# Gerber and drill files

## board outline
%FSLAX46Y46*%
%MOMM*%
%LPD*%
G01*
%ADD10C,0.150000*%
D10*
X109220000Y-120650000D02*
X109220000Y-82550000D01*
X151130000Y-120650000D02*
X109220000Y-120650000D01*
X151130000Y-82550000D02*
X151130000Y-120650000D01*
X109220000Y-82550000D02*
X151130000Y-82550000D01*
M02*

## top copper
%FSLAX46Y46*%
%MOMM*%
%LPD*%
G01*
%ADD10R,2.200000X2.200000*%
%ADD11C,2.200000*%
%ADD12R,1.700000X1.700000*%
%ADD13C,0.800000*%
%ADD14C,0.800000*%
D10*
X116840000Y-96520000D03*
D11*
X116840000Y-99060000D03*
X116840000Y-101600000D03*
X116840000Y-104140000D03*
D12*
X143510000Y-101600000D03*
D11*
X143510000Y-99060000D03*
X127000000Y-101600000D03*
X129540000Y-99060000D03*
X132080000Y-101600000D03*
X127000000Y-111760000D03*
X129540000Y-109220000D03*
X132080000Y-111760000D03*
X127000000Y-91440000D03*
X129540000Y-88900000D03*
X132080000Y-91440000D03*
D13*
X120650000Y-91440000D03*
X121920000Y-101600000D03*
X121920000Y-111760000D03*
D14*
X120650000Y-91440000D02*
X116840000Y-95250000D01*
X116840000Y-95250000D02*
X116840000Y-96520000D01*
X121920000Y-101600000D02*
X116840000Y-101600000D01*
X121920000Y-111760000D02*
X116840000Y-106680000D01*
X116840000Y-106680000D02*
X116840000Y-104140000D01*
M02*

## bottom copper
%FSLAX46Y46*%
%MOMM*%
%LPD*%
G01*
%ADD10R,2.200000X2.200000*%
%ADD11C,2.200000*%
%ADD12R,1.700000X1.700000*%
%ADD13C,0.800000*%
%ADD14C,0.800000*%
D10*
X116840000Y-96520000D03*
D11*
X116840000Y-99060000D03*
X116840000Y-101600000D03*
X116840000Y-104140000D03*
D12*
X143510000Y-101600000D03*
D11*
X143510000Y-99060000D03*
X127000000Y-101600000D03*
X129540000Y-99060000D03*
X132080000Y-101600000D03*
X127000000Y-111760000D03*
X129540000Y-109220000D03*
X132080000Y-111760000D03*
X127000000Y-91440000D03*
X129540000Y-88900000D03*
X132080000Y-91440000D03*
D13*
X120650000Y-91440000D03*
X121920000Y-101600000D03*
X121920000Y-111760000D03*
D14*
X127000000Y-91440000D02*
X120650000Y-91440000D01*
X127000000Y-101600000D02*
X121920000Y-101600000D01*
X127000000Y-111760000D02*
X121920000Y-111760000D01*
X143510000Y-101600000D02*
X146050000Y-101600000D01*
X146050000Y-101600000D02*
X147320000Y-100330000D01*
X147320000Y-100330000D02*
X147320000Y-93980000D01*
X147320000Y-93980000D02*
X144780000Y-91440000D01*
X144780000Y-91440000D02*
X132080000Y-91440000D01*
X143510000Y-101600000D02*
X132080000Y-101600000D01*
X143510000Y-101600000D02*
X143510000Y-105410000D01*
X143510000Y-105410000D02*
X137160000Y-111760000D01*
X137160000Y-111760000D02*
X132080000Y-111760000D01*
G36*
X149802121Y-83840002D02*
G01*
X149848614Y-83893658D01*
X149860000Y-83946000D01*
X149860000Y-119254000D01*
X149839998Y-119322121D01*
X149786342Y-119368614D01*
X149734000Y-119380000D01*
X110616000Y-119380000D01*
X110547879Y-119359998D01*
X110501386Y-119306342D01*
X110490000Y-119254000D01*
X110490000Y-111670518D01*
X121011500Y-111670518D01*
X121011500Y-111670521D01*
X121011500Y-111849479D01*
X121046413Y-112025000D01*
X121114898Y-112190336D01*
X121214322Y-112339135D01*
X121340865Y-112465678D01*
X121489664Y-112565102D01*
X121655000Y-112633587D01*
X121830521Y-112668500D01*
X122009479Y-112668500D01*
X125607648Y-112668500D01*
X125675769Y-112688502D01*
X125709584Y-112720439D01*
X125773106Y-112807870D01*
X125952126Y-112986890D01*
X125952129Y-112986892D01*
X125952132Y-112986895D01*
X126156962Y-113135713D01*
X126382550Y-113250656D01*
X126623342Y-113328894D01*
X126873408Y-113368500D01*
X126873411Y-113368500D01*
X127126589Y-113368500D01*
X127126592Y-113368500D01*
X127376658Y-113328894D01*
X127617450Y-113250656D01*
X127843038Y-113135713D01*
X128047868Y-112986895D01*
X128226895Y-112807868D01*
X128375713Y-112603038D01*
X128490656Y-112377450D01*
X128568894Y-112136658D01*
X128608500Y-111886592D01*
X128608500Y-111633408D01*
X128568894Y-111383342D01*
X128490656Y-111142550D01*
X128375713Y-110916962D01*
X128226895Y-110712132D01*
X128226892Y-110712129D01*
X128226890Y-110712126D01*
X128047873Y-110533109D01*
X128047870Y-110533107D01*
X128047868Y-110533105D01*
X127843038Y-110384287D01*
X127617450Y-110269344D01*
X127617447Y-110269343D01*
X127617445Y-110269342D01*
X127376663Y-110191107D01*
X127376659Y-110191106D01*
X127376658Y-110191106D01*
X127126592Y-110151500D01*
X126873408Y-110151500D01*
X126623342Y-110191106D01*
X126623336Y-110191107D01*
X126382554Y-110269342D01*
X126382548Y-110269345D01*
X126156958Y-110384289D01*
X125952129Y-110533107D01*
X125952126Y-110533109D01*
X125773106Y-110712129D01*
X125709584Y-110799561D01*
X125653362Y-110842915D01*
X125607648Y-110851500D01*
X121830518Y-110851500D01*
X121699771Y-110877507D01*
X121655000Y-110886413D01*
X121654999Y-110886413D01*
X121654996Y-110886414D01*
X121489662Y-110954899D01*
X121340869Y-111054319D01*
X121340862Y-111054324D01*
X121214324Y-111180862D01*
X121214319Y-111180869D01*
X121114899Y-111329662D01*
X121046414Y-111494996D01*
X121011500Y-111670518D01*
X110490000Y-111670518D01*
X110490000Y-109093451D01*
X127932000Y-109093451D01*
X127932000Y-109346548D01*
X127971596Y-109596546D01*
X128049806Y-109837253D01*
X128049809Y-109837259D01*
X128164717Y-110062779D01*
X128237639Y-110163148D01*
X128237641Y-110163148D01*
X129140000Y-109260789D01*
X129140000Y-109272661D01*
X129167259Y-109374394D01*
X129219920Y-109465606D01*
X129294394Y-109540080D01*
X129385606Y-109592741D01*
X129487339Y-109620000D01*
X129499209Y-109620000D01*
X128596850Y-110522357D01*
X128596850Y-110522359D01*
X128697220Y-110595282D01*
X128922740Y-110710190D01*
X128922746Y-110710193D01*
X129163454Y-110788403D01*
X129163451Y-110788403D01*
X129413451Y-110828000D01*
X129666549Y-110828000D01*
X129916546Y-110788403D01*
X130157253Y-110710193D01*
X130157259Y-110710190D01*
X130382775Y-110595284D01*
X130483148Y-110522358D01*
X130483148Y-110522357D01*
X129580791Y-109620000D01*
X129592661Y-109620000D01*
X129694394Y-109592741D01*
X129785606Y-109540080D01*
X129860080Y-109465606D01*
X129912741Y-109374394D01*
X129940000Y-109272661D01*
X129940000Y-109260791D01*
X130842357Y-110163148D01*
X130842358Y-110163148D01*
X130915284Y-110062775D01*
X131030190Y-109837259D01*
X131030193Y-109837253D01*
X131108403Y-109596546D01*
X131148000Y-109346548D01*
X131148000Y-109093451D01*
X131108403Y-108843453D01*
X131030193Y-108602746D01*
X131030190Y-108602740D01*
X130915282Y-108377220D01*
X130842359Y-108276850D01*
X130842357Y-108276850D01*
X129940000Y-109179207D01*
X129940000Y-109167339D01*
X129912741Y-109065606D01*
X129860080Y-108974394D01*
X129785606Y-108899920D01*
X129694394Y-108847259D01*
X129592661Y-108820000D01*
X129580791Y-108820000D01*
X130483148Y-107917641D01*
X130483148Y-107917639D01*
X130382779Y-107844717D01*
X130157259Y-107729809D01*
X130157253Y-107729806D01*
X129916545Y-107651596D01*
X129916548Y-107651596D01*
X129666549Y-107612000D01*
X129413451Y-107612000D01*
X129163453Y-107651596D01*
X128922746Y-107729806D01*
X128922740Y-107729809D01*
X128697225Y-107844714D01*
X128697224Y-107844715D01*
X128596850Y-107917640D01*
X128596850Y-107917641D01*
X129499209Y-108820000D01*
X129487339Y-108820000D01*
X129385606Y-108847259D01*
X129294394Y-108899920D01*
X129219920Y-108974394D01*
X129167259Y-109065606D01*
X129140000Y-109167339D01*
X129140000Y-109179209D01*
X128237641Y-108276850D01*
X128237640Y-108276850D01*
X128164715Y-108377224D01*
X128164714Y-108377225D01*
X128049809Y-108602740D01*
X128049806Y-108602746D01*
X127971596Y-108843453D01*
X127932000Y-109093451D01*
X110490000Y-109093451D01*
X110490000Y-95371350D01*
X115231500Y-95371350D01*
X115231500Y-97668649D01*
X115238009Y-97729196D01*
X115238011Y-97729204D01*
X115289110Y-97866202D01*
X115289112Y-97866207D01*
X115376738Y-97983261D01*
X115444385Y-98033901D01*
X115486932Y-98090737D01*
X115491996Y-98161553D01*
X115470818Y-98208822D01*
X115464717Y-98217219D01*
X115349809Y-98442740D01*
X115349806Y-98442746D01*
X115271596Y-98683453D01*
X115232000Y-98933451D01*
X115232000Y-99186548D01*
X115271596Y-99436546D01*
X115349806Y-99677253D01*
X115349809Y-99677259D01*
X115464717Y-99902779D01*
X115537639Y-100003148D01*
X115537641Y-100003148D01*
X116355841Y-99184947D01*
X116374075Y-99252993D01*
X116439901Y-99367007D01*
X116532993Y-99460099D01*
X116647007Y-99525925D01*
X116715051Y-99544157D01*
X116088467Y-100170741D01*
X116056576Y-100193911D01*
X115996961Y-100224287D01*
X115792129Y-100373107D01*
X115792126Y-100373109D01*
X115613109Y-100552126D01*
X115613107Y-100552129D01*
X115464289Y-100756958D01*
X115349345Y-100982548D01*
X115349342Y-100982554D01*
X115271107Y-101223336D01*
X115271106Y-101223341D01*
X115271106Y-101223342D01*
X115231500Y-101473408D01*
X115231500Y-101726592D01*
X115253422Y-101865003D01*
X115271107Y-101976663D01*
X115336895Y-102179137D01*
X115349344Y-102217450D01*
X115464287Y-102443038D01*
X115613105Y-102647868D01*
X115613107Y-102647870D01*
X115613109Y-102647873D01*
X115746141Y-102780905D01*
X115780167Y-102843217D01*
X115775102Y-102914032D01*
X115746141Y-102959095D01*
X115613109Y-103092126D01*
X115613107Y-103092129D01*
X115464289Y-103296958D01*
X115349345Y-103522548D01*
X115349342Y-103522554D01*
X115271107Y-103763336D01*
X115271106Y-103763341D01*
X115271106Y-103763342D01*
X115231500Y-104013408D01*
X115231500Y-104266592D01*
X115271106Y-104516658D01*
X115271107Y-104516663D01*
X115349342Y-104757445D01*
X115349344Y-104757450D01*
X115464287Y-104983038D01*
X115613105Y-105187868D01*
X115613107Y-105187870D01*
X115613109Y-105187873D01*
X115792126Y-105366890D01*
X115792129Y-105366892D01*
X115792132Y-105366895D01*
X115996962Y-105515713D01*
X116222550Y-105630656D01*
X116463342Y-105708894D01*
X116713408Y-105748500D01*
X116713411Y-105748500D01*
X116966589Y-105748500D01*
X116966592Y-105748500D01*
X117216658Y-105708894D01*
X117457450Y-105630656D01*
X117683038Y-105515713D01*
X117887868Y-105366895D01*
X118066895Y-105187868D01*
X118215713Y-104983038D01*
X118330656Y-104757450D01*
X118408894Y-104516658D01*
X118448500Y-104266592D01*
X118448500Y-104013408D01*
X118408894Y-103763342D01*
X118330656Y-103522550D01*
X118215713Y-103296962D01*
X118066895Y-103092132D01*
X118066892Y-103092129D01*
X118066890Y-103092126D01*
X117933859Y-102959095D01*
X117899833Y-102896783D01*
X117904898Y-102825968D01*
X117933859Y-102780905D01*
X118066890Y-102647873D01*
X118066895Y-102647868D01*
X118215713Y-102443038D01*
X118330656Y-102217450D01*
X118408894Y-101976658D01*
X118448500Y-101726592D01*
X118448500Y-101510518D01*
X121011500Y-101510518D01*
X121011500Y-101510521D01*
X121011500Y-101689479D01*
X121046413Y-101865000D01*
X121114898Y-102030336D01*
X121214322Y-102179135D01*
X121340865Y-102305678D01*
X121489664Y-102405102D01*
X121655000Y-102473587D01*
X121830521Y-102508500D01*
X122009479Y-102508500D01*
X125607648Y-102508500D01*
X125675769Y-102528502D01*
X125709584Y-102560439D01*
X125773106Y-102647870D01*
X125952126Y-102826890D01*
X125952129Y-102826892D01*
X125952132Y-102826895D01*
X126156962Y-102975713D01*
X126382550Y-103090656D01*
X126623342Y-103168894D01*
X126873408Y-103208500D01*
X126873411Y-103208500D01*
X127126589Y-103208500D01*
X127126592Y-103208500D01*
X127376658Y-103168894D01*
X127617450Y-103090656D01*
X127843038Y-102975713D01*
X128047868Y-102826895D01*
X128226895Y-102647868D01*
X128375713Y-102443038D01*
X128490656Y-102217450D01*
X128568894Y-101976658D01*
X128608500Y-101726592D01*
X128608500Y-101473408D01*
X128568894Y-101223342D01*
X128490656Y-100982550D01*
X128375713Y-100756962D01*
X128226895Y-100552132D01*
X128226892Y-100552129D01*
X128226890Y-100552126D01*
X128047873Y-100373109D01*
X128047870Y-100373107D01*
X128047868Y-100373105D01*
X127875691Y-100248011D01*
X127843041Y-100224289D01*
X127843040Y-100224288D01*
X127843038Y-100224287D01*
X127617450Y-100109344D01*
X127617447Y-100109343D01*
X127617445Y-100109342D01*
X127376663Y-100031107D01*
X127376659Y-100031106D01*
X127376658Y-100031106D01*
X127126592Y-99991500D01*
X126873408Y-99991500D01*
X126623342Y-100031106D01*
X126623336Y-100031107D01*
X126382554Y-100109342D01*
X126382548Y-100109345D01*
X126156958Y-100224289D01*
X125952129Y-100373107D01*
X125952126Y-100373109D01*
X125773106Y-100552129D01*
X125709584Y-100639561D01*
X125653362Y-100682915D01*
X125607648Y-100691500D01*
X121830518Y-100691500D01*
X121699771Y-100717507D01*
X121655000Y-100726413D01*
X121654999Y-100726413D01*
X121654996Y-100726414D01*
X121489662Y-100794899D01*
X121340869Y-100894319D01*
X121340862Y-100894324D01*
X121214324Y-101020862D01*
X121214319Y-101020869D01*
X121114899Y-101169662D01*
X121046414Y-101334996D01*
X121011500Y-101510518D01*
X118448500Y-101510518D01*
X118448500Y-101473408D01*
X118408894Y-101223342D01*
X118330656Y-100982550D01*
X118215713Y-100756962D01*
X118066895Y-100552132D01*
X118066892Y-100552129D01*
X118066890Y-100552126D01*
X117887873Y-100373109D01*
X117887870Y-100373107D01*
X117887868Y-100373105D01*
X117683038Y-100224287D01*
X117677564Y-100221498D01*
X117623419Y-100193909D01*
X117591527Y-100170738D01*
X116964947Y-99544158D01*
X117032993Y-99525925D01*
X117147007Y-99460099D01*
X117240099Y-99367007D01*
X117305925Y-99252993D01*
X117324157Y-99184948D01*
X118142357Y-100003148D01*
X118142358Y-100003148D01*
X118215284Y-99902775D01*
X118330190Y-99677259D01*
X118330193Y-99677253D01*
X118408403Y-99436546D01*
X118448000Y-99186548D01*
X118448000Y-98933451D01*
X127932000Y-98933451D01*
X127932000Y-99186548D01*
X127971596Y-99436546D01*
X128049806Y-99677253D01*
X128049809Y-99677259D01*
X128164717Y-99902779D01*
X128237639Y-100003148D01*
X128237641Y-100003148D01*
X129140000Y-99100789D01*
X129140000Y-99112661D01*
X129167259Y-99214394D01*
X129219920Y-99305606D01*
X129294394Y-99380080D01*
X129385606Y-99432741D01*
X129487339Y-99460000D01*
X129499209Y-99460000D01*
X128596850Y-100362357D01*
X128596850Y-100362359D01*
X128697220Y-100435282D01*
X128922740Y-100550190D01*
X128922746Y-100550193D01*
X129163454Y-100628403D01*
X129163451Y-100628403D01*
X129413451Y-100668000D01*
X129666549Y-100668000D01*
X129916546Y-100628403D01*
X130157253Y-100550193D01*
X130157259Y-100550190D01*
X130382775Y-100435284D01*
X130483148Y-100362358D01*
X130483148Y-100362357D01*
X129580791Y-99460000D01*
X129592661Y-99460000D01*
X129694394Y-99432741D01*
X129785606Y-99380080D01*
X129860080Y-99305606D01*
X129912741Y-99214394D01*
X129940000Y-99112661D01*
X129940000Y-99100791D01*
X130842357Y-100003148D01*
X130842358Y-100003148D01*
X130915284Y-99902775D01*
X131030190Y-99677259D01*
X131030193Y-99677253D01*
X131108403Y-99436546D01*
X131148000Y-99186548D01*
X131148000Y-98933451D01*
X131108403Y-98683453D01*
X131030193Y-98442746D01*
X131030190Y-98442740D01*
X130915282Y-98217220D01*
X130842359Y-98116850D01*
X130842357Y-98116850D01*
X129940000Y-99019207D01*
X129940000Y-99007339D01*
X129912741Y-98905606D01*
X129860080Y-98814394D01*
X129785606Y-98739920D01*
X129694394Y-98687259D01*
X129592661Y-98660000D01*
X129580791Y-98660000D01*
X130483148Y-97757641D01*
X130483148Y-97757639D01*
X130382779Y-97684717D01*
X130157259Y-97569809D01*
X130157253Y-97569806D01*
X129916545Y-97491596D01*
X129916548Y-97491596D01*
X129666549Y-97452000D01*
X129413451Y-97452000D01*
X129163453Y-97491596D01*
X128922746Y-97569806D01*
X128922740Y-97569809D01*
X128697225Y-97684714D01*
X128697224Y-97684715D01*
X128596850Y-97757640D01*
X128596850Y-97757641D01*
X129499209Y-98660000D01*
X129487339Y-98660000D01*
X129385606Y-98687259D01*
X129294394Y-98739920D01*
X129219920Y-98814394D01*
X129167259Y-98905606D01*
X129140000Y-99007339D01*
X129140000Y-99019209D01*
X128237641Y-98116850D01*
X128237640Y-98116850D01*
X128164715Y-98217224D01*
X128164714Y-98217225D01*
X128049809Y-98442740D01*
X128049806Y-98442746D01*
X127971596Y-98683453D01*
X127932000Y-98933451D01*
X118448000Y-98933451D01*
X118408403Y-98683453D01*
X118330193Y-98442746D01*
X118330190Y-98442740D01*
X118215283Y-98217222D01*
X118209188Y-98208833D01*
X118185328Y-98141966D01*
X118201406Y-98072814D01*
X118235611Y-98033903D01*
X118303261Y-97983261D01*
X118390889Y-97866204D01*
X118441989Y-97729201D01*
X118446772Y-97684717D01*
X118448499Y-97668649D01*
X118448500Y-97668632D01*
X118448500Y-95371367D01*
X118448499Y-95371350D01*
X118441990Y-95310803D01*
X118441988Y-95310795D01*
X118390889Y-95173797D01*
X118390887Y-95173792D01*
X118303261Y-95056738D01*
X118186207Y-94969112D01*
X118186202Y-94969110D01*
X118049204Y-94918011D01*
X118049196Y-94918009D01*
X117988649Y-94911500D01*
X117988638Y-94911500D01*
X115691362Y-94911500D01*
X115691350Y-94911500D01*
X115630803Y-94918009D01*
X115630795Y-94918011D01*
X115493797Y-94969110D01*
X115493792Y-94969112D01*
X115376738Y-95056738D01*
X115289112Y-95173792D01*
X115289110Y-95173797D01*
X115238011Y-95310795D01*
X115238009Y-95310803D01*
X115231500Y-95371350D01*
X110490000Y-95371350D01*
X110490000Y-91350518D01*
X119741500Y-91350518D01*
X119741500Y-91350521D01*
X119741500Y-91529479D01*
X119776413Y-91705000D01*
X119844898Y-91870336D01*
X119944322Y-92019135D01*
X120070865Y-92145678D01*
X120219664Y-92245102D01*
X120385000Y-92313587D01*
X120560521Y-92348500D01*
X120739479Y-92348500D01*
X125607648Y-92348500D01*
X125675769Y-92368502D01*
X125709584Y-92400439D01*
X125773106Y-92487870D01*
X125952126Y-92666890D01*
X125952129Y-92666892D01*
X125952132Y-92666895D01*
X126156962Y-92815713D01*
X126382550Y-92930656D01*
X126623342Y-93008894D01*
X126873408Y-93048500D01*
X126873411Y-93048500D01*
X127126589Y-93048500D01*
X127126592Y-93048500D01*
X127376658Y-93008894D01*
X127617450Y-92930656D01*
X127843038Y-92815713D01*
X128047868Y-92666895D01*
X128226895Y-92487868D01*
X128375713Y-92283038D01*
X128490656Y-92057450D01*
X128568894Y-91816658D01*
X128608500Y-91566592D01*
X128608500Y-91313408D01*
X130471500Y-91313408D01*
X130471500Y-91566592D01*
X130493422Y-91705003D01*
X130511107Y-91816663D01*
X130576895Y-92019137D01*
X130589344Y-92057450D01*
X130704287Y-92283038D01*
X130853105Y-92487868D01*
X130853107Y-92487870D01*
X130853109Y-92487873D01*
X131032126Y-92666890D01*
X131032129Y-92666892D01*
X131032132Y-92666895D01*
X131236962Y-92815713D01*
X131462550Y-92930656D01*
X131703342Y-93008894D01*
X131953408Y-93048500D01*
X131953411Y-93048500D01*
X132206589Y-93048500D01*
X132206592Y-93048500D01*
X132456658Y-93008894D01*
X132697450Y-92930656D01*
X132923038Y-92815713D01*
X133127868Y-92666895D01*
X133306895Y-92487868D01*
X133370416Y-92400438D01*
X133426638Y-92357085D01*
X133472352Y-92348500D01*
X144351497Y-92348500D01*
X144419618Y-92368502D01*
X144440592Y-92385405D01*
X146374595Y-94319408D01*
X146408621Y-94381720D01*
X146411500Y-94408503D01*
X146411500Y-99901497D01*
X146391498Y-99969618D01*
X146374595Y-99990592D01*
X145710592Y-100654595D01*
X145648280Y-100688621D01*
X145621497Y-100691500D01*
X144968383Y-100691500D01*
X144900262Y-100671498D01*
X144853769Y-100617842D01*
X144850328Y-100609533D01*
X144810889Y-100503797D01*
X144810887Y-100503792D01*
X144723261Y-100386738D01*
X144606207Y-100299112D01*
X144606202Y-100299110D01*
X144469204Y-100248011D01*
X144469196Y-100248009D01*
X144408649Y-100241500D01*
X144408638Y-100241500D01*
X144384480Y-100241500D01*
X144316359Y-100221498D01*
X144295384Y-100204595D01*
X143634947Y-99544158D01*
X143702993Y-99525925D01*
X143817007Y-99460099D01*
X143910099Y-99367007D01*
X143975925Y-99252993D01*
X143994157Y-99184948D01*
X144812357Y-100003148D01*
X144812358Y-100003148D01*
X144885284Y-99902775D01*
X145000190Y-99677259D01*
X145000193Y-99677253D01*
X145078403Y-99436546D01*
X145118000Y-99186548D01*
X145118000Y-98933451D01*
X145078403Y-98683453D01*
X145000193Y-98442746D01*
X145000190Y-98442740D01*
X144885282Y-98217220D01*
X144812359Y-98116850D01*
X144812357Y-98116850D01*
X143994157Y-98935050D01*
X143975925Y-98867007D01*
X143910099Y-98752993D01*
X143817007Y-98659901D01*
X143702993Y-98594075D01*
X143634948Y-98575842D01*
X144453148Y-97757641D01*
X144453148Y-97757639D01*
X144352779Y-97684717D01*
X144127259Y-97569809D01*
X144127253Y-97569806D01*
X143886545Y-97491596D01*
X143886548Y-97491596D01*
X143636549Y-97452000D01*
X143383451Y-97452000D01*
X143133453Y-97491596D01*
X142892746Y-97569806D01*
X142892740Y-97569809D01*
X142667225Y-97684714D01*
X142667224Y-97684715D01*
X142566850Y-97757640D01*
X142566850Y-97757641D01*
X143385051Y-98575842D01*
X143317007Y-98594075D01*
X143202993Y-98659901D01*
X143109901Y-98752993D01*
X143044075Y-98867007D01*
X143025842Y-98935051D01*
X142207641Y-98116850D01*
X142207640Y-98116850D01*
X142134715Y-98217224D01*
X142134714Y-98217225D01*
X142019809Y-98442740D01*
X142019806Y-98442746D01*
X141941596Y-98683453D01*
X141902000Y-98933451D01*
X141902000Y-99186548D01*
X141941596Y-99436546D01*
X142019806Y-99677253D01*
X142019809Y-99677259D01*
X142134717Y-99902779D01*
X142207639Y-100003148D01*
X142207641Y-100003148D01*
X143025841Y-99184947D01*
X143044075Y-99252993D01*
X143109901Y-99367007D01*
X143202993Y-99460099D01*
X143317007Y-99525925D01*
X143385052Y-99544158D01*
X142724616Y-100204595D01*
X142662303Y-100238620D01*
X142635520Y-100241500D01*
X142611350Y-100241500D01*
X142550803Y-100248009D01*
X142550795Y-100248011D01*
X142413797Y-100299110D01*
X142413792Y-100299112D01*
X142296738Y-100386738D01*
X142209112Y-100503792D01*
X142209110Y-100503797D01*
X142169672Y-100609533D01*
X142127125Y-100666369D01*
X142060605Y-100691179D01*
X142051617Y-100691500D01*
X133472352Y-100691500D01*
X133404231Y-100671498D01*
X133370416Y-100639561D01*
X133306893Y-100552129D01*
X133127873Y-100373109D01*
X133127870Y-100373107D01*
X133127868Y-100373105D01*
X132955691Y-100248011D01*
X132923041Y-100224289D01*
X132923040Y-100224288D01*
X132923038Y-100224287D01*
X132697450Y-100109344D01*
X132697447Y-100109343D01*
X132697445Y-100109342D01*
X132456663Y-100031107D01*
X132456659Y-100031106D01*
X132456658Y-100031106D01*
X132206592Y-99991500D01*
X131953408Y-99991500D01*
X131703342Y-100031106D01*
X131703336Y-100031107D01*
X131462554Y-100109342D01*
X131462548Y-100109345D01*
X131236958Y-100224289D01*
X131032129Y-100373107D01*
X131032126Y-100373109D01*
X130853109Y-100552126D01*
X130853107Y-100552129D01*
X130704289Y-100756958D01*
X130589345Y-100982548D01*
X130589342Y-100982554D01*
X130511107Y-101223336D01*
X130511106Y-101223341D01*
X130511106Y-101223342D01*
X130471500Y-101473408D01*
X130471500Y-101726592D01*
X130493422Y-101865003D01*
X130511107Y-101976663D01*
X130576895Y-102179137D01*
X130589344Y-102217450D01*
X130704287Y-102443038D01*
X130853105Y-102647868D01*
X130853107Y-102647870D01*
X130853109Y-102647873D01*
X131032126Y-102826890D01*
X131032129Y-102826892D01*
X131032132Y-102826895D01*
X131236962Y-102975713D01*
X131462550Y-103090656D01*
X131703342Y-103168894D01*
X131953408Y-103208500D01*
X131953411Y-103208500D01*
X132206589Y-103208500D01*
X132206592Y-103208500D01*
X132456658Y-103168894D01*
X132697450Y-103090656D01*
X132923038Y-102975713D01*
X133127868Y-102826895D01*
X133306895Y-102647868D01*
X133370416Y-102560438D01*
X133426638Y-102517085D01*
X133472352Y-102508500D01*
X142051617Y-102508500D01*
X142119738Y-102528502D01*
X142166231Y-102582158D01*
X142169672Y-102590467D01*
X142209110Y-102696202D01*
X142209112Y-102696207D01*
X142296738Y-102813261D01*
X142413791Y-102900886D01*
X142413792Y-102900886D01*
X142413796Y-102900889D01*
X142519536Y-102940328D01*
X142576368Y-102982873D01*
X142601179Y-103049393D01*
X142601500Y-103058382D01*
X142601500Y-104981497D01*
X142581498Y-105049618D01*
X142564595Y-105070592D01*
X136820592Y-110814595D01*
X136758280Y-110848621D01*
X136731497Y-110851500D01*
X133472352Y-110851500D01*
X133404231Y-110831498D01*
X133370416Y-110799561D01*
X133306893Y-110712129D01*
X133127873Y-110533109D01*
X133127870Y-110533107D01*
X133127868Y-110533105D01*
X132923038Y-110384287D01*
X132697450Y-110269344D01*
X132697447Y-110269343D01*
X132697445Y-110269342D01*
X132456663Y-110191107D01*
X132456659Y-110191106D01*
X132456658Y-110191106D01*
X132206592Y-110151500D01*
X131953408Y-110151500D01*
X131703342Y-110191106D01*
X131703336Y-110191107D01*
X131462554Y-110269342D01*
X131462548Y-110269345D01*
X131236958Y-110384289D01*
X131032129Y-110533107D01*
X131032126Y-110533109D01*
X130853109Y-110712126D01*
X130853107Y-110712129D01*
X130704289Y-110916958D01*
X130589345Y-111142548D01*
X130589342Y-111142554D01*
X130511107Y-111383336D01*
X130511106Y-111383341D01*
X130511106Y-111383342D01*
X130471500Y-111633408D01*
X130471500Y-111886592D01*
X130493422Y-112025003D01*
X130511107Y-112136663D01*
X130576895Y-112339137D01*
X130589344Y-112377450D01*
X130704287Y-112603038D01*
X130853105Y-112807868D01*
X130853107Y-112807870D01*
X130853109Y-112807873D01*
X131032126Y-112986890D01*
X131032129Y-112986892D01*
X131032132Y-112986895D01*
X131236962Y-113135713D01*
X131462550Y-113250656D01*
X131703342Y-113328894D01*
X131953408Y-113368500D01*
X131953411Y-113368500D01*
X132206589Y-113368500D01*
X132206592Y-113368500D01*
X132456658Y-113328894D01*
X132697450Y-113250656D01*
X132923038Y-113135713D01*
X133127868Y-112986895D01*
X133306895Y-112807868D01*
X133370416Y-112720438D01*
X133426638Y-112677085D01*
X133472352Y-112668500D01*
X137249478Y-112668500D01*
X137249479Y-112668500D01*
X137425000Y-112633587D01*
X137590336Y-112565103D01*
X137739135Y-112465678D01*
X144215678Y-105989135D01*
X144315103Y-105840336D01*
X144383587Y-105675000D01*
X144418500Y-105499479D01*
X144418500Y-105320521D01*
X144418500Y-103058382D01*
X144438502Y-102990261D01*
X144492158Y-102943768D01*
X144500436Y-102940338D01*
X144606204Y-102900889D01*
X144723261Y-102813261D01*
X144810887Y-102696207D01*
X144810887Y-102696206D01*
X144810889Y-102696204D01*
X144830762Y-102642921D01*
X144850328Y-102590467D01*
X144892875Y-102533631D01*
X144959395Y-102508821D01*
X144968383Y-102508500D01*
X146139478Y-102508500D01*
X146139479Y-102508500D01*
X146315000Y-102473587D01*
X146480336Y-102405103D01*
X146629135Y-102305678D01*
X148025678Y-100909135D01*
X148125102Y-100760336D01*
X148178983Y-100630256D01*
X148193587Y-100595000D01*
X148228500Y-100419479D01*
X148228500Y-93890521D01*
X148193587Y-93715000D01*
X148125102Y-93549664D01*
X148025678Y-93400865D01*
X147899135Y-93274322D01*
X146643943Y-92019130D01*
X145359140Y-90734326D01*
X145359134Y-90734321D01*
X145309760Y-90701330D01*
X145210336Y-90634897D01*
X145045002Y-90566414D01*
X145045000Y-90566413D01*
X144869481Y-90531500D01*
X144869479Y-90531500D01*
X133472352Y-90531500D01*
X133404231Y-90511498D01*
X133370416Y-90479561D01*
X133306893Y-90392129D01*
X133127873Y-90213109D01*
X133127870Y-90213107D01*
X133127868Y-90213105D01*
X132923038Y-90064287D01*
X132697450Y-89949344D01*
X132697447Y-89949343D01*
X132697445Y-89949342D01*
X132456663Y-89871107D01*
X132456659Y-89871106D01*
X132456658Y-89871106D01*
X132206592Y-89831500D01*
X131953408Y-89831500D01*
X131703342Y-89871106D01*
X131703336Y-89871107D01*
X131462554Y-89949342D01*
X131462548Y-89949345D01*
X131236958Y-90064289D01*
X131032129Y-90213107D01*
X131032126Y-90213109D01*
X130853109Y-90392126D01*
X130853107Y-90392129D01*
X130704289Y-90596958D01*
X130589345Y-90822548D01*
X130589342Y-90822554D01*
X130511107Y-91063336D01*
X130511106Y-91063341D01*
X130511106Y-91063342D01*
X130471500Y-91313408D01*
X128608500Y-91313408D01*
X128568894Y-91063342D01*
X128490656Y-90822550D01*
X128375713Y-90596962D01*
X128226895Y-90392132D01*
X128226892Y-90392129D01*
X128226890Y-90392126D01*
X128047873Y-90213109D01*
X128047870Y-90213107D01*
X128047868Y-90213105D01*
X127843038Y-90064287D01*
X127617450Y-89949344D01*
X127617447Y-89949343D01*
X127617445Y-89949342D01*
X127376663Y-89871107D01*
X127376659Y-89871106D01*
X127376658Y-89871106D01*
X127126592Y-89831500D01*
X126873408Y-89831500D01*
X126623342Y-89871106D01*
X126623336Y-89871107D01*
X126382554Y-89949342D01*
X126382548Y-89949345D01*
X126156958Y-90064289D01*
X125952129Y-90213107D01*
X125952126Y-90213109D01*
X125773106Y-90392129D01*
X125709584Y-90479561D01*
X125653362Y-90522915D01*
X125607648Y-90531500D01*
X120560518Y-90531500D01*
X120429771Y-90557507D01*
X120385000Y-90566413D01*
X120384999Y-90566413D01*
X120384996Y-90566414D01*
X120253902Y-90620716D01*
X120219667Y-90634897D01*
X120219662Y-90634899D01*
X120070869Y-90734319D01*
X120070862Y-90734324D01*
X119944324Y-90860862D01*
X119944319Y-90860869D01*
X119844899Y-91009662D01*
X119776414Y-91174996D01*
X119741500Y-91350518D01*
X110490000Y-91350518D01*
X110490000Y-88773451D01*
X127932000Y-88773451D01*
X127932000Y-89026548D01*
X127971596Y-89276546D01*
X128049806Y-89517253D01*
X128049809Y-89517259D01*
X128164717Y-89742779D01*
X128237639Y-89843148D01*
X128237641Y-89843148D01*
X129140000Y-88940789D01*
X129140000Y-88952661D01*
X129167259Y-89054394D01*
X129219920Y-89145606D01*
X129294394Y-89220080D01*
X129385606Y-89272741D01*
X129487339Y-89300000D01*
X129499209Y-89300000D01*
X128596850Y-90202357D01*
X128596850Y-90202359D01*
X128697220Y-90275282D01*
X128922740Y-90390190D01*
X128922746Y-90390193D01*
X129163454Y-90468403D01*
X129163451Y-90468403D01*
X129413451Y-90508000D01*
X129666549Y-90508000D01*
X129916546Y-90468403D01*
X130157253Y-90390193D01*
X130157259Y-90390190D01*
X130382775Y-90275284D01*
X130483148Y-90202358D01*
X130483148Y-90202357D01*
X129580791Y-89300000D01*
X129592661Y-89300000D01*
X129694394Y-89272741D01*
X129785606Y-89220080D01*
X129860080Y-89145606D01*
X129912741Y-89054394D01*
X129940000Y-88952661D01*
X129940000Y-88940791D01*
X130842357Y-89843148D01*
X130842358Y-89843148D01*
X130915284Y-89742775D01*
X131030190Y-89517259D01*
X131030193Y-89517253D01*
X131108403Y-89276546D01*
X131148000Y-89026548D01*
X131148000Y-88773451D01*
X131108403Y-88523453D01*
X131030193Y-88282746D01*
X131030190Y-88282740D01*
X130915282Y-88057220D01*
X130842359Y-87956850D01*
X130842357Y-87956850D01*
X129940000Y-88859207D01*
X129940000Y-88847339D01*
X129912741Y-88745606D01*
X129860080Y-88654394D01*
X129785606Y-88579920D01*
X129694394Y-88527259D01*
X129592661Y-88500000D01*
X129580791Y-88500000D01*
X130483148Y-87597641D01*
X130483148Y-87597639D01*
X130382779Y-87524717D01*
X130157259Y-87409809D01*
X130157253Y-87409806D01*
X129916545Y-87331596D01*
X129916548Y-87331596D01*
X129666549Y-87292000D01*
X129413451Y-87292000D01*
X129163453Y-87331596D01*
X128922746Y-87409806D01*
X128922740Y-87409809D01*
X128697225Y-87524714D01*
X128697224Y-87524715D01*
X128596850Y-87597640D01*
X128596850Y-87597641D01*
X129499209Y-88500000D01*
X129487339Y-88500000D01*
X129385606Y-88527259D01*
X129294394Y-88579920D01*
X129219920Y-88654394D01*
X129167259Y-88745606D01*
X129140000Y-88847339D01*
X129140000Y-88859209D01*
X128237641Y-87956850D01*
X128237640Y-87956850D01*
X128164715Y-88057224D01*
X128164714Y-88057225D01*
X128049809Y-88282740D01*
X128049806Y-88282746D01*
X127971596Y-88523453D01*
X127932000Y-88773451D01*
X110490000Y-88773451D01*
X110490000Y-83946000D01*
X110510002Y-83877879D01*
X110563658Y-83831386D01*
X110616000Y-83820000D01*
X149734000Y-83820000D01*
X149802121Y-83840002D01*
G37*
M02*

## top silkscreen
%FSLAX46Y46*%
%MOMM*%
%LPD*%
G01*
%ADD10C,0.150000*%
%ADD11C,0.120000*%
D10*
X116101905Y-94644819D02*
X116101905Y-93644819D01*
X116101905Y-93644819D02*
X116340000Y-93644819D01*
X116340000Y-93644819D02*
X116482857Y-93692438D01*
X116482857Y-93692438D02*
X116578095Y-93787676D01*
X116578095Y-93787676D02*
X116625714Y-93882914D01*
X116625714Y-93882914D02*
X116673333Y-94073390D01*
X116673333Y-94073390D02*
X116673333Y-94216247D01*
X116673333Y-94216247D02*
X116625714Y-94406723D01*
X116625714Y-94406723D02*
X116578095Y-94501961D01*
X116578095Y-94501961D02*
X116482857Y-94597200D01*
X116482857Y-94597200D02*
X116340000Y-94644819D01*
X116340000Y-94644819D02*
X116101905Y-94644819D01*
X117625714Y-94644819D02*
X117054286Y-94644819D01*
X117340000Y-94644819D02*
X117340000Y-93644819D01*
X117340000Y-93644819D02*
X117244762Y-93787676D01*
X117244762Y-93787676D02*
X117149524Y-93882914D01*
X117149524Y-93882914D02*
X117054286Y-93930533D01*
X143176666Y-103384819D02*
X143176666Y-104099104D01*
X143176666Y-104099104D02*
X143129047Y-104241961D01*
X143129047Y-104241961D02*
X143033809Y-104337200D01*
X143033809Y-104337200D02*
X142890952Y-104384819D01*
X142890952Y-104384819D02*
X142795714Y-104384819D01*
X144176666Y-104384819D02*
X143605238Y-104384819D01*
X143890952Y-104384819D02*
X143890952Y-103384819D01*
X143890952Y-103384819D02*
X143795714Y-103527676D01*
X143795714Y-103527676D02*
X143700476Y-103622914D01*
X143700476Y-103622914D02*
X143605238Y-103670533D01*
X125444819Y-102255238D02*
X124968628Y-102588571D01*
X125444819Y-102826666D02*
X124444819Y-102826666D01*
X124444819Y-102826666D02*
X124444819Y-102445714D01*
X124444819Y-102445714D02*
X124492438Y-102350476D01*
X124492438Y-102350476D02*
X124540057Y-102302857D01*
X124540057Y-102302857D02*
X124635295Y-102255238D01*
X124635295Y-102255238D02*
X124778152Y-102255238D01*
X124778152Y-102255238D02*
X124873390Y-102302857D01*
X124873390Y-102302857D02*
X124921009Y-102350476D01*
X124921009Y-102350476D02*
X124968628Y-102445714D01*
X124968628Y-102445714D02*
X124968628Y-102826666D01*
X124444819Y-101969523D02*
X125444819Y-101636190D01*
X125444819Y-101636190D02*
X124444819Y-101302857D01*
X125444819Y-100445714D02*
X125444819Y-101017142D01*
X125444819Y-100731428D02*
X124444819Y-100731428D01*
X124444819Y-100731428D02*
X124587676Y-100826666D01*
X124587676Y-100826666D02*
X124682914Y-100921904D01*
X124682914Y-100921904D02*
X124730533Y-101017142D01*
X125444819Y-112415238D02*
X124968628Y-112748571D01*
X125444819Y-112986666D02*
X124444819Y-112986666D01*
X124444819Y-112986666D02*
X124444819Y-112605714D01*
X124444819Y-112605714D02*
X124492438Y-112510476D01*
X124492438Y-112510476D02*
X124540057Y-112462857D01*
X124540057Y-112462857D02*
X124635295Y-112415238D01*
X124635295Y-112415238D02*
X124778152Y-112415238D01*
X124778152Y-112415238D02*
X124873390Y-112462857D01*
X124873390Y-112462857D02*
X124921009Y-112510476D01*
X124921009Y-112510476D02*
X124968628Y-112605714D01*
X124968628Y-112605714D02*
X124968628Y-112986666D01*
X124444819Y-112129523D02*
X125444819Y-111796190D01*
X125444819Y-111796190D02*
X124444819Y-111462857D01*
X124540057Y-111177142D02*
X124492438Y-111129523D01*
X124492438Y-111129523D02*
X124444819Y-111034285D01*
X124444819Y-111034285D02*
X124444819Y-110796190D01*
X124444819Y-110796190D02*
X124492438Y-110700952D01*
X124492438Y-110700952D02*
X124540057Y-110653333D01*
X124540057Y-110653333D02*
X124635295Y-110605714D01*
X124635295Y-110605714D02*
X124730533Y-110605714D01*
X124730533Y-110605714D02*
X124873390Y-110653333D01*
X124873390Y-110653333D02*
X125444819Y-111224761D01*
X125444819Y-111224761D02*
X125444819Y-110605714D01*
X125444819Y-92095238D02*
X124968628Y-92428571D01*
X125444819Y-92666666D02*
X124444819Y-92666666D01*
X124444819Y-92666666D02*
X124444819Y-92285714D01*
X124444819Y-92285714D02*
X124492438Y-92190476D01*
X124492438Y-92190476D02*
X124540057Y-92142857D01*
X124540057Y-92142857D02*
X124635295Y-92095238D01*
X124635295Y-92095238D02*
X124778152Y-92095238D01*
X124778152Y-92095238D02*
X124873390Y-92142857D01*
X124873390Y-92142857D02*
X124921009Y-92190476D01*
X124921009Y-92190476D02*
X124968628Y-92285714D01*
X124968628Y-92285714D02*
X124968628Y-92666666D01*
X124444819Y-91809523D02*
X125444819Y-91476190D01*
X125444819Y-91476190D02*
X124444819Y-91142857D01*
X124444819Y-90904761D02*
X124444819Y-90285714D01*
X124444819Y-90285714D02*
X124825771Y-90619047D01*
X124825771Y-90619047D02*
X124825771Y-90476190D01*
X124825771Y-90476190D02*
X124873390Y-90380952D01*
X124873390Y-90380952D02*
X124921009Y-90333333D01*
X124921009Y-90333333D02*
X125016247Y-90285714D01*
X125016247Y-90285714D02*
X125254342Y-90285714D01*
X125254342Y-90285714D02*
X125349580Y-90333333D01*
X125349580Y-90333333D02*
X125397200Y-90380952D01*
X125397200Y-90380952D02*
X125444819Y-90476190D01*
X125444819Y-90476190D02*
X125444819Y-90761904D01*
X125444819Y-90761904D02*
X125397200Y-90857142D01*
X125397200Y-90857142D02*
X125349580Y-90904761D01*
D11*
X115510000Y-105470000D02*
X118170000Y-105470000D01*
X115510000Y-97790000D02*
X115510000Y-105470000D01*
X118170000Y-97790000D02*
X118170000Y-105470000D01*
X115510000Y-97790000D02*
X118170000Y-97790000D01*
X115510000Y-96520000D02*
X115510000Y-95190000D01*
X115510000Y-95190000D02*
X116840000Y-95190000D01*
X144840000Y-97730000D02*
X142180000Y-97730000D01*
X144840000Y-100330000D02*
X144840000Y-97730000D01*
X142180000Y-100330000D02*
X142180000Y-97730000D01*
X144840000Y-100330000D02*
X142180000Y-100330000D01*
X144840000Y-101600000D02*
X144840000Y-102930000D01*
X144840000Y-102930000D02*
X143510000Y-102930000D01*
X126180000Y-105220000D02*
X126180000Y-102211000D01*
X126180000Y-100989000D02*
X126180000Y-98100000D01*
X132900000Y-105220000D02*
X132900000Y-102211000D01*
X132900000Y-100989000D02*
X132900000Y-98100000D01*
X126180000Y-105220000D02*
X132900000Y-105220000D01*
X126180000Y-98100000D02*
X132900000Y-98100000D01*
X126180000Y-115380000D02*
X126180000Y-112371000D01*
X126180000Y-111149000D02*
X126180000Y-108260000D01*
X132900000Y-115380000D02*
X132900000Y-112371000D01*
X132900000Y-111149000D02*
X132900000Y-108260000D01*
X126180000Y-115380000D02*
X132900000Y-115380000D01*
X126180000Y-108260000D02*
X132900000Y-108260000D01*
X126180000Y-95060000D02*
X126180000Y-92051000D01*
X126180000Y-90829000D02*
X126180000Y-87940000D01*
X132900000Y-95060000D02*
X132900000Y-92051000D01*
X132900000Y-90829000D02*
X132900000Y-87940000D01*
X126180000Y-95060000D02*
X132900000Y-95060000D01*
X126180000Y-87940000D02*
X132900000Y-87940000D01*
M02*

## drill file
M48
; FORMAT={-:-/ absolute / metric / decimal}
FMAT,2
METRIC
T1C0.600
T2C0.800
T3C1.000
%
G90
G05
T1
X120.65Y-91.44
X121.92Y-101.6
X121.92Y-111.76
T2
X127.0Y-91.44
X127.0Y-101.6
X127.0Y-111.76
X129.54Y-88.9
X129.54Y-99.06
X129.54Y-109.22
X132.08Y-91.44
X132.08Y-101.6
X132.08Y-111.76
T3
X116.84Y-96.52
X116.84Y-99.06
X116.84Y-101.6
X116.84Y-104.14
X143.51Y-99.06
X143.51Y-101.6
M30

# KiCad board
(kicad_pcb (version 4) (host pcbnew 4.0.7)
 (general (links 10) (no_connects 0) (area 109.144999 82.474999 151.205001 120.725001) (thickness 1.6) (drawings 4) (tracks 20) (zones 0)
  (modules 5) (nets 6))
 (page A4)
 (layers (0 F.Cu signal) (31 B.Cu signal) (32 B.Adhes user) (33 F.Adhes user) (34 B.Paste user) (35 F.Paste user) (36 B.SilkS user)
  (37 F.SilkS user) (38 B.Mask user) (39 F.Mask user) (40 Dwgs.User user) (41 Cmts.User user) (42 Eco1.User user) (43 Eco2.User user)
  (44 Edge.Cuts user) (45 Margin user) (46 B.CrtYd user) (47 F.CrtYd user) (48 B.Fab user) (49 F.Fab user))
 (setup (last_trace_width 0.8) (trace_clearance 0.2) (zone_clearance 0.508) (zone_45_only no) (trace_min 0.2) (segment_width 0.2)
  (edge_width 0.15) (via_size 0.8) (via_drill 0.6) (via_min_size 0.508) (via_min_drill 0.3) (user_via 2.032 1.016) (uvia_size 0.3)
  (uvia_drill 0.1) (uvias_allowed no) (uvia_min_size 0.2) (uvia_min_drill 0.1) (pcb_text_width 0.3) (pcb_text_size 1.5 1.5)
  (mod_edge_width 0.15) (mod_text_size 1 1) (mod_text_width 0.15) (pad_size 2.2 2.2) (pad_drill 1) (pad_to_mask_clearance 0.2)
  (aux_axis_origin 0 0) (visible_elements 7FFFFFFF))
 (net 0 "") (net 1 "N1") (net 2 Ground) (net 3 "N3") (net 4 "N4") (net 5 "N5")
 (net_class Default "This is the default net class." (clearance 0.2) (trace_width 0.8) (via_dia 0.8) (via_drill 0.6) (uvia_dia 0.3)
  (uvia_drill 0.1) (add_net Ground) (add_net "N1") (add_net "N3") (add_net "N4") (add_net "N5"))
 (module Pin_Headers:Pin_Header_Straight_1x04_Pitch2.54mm (layer F.Cu) (at 116.84 96.52)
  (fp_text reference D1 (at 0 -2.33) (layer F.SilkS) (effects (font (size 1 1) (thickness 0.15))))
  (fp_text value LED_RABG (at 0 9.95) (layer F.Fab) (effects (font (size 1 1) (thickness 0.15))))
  (fp_line (start -1.33 8.95) (end 1.33 8.95) (layer F.SilkS) (width 0.12))
  (fp_line (start -1.33 1.27) (end -1.33 8.95) (layer F.SilkS) (width 0.12))
  (fp_line (start 1.33 1.27) (end 1.33 8.95) (layer F.SilkS) (width 0.12))
  (fp_line (start -1.33 1.27) (end 1.33 1.27) (layer F.SilkS) (width 0.12))
  (fp_line (start -1.33 0) (end -1.33 -1.33) (layer F.SilkS) (width 0.12))
  (fp_line (start -1.33 -1.33) (end 0 -1.33) (layer F.SilkS) (width 0.12))
  (pad 1 thru_hole rect (at 0 0) (size 2.2 2.2) (drill 1) (layers *.Cu *.Mask) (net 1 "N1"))
  (pad 2 thru_hole circle (at 0 2.54) (size 2.2 2.2) (drill 1) (layers *.Cu *.Mask) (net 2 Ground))
  (pad 3 thru_hole circle (at 0 5.08) (size 2.2 2.2) (drill 1) (layers *.Cu *.Mask) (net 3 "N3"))
  (pad 4 thru_hole circle (at 0 7.62) (size 2.2 2.2) (drill 1) (layers *.Cu *.Mask) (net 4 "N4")))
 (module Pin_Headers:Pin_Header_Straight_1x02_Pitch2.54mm (layer F.Cu) (at 143.51 101.6 180)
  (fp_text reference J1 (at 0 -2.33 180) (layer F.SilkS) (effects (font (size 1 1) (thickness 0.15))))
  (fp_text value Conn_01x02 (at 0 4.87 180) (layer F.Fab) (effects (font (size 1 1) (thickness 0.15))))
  (fp_line (start -1.33 3.87) (end 1.33 3.87) (layer F.SilkS) (width 0.12))
  (fp_line (start -1.33 1.27) (end -1.33 3.87) (layer F.SilkS) (width 0.12))
  (fp_line (start 1.33 1.27) (end 1.33 3.87) (layer F.SilkS) (width 0.12))
  (fp_line (start -1.33 1.27) (end 1.33 1.27) (layer F.SilkS) (width 0.12))
  (fp_line (start -1.33 0) (end -1.33 -1.33) (layer F.SilkS) (width 0.12))
  (fp_line (start -1.33 -1.33) (end 0 -1.33) (layer F.SilkS) (width 0.12))
  (pad 1 thru_hole rect (at 0 0 180) (size 1.7 1.7) (drill 1) (layers *.Cu *.Mask) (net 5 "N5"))
  (pad 2 thru_hole circle (at 0 2.54 180) (size 2.2 2.2) (drill 1) (layers *.Cu *.Mask) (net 2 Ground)))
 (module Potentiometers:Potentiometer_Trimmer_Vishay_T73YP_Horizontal (layer F.Cu) (at 132.08 101.6 90)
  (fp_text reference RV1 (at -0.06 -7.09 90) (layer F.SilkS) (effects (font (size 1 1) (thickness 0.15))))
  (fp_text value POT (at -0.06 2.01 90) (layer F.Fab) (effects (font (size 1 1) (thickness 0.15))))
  (fp_line (start -3.62 -5.9) (end -0.611 -5.9) (layer F.SilkS) (width 0.12))
  (fp_line (start 0.611 -5.9) (end 3.5 -5.9) (layer F.SilkS) (width 0.12))
  (fp_line (start -3.62 0.82) (end -0.611 0.82) (layer F.SilkS) (width 0.12))
  (fp_line (start 0.611 0.82) (end 3.5 0.82) (layer F.SilkS) (width 0.12))
  (fp_line (start -3.62 -5.9) (end -3.62 0.82) (layer F.SilkS) (width 0.12))
  (fp_line (start 3.5 -5.9) (end 3.5 0.82) (layer F.SilkS) (width 0.12))
  (pad 3 thru_hole circle (at 0 -5.08 90) (size 2.2 2.2) (drill 0.8) (layers *.Cu *.Mask) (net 3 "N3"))
  (pad 2 thru_hole circle (at 2.54 -2.54 90) (size 2.2 2.2) (drill 0.8) (layers *.Cu *.Mask) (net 2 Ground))
  (pad 1 thru_hole circle (at 0 0 90) (size 2.2 2.2) (drill 0.8) (layers *.Cu *.Mask) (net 5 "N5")))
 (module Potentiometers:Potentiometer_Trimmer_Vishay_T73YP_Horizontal (layer F.Cu) (at 132.08 111.76 90)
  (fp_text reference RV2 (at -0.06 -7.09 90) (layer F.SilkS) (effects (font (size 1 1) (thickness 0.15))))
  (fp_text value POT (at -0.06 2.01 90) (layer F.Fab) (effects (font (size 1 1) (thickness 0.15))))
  (fp_line (start -3.62 -5.9) (end -0.611 -5.9) (layer F.SilkS) (width 0.12))
  (fp_line (start 0.611 -5.9) (end 3.5 -5.9) (layer F.SilkS) (width 0.12))
  (fp_line (start -3.62 0.82) (end -0.611 0.82) (layer F.SilkS) (width 0.12))
  (fp_line (start 0.611 0.82) (end 3.5 0.82) (layer F.SilkS) (width 0.12))
  (fp_line (start -3.62 -5.9) (end -3.62 0.82) (layer F.SilkS) (width 0.12))
  (fp_line (start 3.5 -5.9) (end 3.5 0.82) (layer F.SilkS) (width 0.12))
  (pad 3 thru_hole circle (at 0 -5.08 90) (size 2.2 2.2) (drill 0.8) (layers *.Cu *.Mask) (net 4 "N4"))
  (pad 2 thru_hole circle (at 2.54 -2.54 90) (size 2.2 2.2) (drill 0.8) (layers *.Cu *.Mask) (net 2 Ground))
  (pad 1 thru_hole circle (at 0 0 90) (size 2.2 2.2) (drill 0.8) (layers *.Cu *.Mask) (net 5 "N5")))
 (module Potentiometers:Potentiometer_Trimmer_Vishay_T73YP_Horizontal (layer F.Cu) (at 132.08 91.44 90)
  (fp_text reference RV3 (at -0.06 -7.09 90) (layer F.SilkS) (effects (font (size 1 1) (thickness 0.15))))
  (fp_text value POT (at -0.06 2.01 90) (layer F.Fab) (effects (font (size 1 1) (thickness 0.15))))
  (fp_line (start -3.62 -5.9) (end -0.611 -5.9) (layer F.SilkS) (width 0.12))
  (fp_line (start 0.611 -5.9) (end 3.5 -5.9) (layer F.SilkS) (width 0.12))
  (fp_line (start -3.62 0.82) (end -0.611 0.82) (layer F.SilkS) (width 0.12))
  (fp_line (start 0.611 0.82) (end 3.5 0.82) (layer F.SilkS) (width 0.12))
  (fp_line (start -3.62 -5.9) (end -3.62 0.82) (layer F.SilkS) (width 0.12))
  (fp_line (start 3.5 -5.9) (end 3.5 0.82) (layer F.SilkS) (width 0.12))
  (pad 3 thru_hole circle (at 0 -5.08 90) (size 2.2 2.2) (drill 0.8) (layers *.Cu *.Mask) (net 1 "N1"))
  (pad 2 thru_hole circle (at 2.54 -2.54 90) (size 2.2 2.2) (drill 0.8) (layers *.Cu *.Mask) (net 2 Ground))
  (pad 1 thru_hole circle (at 0 0 90) (size 2.2 2.2) (drill 0.8) (layers *.Cu *.Mask) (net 5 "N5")))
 (gr_line (start 109.22 120.65) (end 109.22 82.55) (angle 90) (layer Edge.Cuts) (width 0.15))
 (gr_line (start 151.13 120.65) (end 109.22 120.65) (angle 90) (layer Edge.Cuts) (width 0.15))
 (gr_line (start 151.13 82.55) (end 151.13 120.65) (angle 90) (layer Edge.Cuts) (width 0.15))
 (gr_line (start 109.22 82.55) (end 151.13 82.55) (angle 90) (layer Edge.Cuts) (width 0.15))
 (segment (start 127 91.44) (end 120.65 91.44) (width 0.8) (layer B.Cu) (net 1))
 (via (at 120.65 91.44) (size 0.8) (drill 0.6) (layers F.Cu B.Cu) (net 1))
 (segment (start 120.65 91.44) (end 116.84 95.25) (width 0.8) (layer F.Cu) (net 1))
 (segment (start 116.84 95.25) (end 116.84 96.52) (width 0.8) (layer F.Cu) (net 1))
 (segment (start 127 101.6) (end 121.92 101.6) (width 0.8) (layer B.Cu) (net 3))
 (via (at 121.92 101.6) (size 0.8) (drill 0.6) (layers F.Cu B.Cu) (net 3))
 (segment (start 121.92 101.6) (end 116.84 101.6) (width 0.8) (layer F.Cu) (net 3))
 (segment (start 127 111.76) (end 121.92 111.76) (width 0.8) (layer B.Cu) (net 4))
 (via (at 121.92 111.76) (size 0.8) (drill 0.6) (layers F.Cu B.Cu) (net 4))
 (segment (start 121.92 111.76) (end 116.84 106.68) (width 0.8) (layer F.Cu) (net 4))
 (segment (start 116.84 106.68) (end 116.84 104.14) (width 0.8) (layer F.Cu) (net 4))
 (segment (start 143.51 101.6) (end 146.05 101.6) (width 0.8) (layer B.Cu) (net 5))
 (segment (start 146.05 101.6) (end 147.32 100.33) (width 0.8) (layer B.Cu) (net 5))
 (segment (start 147.32 100.33) (end 147.32 93.98) (width 0.8) (layer B.Cu) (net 5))
 (segment (start 147.32 93.98) (end 144.78 91.44) (width 0.8) (layer B.Cu) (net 5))
 (segment (start 144.78 91.44) (end 132.08 91.44) (width 0.8) (layer B.Cu) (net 5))
 (segment (start 143.51 101.6) (end 132.08 101.6) (width 0.8) (layer B.Cu) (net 5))
 (segment (start 143.51 101.6) (end 143.51 105.41) (width 0.8) (layer B.Cu) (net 5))
 (segment (start 143.51 105.41) (end 137.16 111.76) (width 0.8) (layer B.Cu) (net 5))
 (segment (start 137.16 111.76) (end 132.08 111.76) (width 0.8) (layer B.Cu) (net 5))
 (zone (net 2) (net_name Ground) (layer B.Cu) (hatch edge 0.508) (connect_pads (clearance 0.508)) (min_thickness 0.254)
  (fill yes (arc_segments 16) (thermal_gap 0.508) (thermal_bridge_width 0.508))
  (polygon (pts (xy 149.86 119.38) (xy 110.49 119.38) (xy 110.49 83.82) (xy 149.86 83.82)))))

